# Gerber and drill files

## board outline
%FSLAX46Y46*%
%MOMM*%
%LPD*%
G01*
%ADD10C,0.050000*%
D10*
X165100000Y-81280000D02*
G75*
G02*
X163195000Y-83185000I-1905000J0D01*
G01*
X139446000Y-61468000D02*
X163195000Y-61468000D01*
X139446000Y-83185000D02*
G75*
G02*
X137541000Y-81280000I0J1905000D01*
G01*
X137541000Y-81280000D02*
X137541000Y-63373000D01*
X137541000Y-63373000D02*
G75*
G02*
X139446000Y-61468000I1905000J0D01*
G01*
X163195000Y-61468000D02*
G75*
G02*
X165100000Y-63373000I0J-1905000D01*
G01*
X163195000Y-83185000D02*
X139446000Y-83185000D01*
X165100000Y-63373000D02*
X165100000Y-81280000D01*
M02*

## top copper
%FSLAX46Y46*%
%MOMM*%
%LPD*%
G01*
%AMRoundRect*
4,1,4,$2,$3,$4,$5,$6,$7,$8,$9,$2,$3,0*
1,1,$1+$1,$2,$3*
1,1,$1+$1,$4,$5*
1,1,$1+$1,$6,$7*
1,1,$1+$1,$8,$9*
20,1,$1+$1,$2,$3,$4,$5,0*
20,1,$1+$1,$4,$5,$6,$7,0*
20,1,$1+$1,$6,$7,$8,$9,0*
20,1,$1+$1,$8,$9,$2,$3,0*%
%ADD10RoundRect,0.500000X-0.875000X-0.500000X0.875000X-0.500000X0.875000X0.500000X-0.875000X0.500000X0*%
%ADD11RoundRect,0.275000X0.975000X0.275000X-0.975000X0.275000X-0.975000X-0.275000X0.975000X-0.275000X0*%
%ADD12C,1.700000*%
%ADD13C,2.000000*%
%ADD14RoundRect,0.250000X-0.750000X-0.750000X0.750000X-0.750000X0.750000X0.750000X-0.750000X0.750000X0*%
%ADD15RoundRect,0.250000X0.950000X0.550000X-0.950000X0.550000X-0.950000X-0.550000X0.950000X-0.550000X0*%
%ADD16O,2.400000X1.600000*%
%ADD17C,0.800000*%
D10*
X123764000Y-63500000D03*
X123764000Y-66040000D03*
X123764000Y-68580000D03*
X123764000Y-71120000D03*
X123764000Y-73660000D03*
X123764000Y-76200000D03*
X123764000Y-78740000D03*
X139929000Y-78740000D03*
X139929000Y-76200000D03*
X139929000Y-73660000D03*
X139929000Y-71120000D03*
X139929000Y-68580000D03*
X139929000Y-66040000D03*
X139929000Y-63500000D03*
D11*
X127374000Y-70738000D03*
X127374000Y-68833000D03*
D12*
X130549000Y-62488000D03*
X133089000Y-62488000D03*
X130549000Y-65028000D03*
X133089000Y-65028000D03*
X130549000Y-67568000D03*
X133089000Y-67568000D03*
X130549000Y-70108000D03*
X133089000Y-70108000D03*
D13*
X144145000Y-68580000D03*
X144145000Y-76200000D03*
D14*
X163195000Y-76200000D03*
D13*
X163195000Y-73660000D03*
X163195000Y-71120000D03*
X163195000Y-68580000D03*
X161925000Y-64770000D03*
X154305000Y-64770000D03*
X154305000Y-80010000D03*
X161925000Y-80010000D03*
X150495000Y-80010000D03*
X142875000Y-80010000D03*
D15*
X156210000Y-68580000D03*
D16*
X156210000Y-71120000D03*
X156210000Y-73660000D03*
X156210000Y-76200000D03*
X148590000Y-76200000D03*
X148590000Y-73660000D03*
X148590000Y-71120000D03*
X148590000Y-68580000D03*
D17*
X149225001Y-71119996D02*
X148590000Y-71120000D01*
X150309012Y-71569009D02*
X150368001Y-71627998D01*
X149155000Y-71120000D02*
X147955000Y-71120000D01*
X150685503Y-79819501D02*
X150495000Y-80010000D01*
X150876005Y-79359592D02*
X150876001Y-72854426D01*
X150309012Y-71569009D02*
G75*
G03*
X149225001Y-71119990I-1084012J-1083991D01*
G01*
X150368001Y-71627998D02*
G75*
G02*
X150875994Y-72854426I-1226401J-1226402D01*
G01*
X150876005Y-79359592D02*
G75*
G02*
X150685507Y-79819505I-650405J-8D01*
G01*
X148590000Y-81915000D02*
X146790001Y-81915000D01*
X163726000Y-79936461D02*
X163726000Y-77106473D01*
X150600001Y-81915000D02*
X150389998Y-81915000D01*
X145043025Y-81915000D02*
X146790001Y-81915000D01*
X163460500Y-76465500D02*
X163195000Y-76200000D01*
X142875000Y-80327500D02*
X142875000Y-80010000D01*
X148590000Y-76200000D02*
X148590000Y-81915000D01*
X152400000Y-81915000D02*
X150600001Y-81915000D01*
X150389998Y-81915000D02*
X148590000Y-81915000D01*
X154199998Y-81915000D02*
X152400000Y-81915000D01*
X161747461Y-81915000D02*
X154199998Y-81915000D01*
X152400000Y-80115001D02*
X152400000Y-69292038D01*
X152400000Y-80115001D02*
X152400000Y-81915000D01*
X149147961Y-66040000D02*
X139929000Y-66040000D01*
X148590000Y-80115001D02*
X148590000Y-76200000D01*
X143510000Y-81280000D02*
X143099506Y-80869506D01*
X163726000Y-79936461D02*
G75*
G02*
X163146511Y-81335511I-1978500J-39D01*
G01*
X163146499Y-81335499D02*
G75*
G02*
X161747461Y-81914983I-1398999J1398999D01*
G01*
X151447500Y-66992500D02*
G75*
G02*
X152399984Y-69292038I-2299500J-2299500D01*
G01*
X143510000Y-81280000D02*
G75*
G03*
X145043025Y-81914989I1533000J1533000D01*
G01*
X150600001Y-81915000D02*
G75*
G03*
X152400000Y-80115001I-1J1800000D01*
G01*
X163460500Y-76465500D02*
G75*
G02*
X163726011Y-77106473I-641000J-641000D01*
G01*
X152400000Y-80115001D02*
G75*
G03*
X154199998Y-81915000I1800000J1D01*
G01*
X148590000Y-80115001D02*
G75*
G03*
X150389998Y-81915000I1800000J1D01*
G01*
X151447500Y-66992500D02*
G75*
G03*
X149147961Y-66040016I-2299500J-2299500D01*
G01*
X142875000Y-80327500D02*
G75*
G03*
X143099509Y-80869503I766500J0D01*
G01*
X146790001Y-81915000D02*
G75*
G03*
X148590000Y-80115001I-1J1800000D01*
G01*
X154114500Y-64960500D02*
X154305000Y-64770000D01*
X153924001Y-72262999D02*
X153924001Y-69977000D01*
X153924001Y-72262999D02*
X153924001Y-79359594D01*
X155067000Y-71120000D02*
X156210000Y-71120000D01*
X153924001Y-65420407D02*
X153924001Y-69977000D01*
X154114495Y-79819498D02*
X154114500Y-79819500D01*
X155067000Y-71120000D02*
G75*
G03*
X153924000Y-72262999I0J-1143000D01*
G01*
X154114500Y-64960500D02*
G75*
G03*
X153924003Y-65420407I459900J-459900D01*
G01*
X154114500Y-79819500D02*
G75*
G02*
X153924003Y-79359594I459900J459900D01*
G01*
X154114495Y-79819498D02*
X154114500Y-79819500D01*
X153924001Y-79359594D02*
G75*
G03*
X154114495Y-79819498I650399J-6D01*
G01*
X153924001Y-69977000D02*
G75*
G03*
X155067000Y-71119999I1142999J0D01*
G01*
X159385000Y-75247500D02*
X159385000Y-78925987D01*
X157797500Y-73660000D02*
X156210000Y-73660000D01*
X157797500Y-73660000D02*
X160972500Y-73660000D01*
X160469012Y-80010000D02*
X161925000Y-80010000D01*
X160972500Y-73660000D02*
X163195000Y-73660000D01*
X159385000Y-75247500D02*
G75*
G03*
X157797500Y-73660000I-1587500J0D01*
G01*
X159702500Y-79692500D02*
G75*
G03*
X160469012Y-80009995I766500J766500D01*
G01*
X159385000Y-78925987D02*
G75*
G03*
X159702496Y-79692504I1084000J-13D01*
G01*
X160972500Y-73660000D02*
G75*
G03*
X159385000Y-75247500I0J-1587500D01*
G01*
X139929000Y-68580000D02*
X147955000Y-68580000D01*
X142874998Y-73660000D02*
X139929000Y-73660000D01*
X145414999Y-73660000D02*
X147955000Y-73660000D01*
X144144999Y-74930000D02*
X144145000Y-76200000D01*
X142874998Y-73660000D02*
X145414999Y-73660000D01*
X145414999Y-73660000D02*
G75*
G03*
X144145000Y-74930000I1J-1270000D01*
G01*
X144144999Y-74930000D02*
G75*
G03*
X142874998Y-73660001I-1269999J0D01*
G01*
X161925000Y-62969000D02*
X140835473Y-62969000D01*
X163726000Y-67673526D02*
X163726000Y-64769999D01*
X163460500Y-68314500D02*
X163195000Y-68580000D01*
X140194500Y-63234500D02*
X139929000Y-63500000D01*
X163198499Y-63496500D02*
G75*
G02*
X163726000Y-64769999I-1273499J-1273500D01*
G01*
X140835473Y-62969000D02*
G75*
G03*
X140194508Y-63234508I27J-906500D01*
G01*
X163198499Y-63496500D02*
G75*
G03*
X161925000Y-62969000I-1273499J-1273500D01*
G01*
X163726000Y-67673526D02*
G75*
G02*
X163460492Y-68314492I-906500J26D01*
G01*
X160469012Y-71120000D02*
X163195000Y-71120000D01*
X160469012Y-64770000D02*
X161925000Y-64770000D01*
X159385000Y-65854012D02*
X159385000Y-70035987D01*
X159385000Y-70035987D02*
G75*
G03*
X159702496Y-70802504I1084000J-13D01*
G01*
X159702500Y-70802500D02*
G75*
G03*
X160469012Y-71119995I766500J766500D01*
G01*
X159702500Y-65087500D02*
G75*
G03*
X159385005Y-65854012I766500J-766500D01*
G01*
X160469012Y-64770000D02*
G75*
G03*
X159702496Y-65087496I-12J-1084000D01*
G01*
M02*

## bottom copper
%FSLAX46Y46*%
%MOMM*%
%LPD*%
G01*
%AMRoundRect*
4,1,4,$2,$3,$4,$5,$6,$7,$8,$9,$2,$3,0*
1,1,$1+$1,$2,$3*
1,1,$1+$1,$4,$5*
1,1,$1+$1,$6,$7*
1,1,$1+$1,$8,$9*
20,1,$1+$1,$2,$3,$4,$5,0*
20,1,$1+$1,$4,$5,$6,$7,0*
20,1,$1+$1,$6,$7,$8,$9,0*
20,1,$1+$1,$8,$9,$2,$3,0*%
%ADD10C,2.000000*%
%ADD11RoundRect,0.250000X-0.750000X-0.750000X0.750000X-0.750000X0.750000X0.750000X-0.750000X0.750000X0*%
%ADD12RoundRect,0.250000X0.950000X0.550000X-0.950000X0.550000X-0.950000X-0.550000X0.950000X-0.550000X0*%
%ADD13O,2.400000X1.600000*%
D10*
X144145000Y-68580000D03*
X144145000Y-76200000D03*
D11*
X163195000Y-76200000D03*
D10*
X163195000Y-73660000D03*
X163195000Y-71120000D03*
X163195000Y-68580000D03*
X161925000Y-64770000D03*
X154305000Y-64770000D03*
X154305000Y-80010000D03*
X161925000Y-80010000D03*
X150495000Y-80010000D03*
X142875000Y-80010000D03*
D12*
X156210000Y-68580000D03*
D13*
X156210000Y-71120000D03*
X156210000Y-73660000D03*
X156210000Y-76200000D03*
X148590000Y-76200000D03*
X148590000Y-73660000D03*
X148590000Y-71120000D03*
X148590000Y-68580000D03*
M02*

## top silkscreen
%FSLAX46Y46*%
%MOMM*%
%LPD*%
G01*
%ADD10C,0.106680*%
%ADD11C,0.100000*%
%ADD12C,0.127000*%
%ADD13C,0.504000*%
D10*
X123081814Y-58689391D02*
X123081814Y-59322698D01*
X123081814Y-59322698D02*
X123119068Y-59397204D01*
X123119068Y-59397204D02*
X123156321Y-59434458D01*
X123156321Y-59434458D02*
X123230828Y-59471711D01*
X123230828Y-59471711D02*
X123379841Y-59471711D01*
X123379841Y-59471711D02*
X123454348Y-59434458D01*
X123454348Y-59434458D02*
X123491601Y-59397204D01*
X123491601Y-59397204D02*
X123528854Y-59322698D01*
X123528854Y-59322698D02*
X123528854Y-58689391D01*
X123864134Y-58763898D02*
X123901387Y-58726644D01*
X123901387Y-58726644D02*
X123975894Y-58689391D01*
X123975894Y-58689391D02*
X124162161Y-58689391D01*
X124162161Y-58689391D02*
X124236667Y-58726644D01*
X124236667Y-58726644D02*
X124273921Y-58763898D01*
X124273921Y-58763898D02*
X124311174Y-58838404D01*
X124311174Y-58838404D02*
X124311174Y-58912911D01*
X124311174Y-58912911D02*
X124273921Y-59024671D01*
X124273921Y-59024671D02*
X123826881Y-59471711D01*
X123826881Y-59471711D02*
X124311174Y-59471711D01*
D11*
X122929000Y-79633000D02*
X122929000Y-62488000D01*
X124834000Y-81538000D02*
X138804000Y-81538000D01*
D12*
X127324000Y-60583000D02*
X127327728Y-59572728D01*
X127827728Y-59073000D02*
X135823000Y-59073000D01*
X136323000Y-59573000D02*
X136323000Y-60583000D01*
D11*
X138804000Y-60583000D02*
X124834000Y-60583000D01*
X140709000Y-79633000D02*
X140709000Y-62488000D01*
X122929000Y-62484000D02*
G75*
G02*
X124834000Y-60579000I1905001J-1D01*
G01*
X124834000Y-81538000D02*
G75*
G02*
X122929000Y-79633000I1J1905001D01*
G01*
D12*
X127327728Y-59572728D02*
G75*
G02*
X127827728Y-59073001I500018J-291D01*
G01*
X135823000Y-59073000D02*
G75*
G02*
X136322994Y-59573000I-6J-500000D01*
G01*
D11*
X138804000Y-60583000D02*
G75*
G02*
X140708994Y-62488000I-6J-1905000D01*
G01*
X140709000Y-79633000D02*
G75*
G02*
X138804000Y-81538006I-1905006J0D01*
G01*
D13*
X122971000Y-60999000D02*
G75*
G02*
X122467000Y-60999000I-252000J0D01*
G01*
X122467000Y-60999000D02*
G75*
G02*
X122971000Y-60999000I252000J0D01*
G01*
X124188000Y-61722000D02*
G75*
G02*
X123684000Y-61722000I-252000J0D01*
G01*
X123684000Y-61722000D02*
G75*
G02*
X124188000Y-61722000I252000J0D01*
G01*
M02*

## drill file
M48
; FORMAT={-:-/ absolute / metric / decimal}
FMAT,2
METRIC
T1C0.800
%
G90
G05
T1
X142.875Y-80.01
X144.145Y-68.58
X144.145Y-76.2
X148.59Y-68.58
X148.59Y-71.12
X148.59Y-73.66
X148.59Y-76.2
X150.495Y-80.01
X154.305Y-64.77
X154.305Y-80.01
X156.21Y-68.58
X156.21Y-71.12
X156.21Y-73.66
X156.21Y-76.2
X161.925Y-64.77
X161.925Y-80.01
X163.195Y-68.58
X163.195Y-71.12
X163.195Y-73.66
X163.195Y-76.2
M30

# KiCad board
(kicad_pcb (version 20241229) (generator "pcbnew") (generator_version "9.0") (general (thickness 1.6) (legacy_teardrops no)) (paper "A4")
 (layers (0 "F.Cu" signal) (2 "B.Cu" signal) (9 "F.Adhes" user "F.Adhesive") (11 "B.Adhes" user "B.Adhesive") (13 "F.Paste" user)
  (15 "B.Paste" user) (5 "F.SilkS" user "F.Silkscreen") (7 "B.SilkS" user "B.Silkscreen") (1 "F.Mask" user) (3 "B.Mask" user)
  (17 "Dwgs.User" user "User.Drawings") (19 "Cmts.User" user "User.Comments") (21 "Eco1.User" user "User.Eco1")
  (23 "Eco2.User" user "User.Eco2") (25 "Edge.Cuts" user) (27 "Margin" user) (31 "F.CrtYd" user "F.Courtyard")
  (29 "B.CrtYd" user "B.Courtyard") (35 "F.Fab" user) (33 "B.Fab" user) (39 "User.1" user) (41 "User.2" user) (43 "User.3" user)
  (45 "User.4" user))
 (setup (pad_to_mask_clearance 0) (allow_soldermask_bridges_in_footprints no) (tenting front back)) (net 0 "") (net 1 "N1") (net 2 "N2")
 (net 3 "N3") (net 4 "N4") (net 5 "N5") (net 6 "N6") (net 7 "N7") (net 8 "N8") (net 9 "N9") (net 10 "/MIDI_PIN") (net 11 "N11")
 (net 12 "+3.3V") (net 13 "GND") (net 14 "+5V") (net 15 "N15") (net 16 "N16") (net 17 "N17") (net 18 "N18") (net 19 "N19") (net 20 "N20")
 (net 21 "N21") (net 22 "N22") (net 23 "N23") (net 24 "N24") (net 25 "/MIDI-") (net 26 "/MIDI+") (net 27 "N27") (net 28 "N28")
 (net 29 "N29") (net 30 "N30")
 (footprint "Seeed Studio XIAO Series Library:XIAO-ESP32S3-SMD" (layer "F.Cu") (at 131.825364 71.073)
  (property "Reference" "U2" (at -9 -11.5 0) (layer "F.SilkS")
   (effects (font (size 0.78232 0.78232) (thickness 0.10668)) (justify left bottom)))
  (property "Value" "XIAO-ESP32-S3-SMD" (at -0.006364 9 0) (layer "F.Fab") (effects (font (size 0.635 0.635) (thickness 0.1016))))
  (fp_line (start -8.896364 8.56) (end -8.896364 -8.585) (stroke (width 0.1) (type solid)) (layer "F.SilkS"))
  (fp_line (start -6.991364 10.465) (end 6.978636 10.465) (stroke (width 0.1) (type solid)) (layer "F.SilkS"))
  (fp_line (start -4.501364 -10.49) (end -4.497636 -11.500272) (stroke (width 0.127) (type solid)) (layer "F.SilkS"))
  (fp_line (start -3.997636 -12) (end 3.997636 -12) (stroke (width 0.127) (type solid)) (layer "F.SilkS"))
  (fp_line (start 4.497636 -11.5) (end 4.497636 -10.49) (stroke (width 0.127) (type solid)) (layer "F.SilkS"))
  (fp_line (start 6.978636 -10.49) (end -6.991364 -10.49) (stroke (width 0.1) (type solid)) (layer "F.SilkS"))
  (fp_line (start 8.883636 8.56) (end 8.883636 -8.585) (stroke (width 0.1) (type solid)) (layer "F.SilkS"))
  (fp_arc (start -8.896364 -8.589) (mid -8.338402 -9.936038) (end -6.991364 -10.494) (stroke (width 0.1) (type solid)) (layer "F.SilkS"))
  (fp_arc (start -6.991364 10.465) (mid -8.338402 9.907038) (end -8.896364 8.56) (stroke (width 0.1) (type solid)) (layer "F.SilkS"))
  (fp_arc (start -4.497636 -11.500272) (mid -4.351088 -11.853644) (end -3.997636 -12) (stroke (width 0.127) (type default))
   (layer "F.SilkS"))
  (fp_arc (start 3.997636 -12) (mid 4.351189 -11.853553) (end 4.497636 -11.5) (stroke (width 0.127) (type default)) (layer "F.SilkS"))
  (fp_arc (start 6.978636 -10.49) (mid 8.325674 -9.932038) (end 8.883636 -8.585) (stroke (width 0.1) (type solid)) (layer "F.SilkS"))
  (fp_arc (start 8.883636 8.56) (mid 8.325674 9.907038) (end 6.978636 10.465) (stroke (width 0.1) (type solid)) (layer "F.SilkS"))
  (fp_circle (center -9.106364 -10.074) (end -9.106364 -10.328) (stroke (width 0.5) (type solid)) (fill yes) (layer "F.SilkS"))
  (fp_circle (center -7.889364 -9.351) (end -7.889364 -9.605) (stroke (width 0.5) (type solid)) (fill yes) (layer "F.SilkS"))
  (pad "1" smd roundrect (at -8.061364 -7.573) (size 2.75 2) (layers "F.Cu" "F.Mask" "F.Paste") (roundrect_rratio 0.25) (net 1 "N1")
   (solder_mask_margin 0.0508) (thermal_bridge_angle 45))
  (pad "2" smd roundrect (at -8.061364 -5.033) (size 2.75 2) (layers "F.Cu" "F.Mask" "F.Paste") (roundrect_rratio 0.25) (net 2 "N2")
   (solder_mask_margin 0.0508) (thermal_bridge_angle 45))
  (pad "3" smd roundrect (at -8.061364 -2.493) (size 2.75 2) (layers "F.Cu" "F.Mask" "F.Paste") (roundrect_rratio 0.25) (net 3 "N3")
   (solder_mask_margin 0.0508) (thermal_bridge_angle 45))
  (pad "4" smd roundrect (at -8.061364 0.047) (size 2.75 2) (layers "F.Cu" "F.Mask" "F.Paste") (roundrect_rratio 0.25) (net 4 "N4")
   (solder_mask_margin 0.0508) (thermal_bridge_angle 45))
  (pad "5" smd roundrect (at -8.061364 2.587) (size 2.75 2) (layers "F.Cu" "F.Mask" "F.Paste") (roundrect_rratio 0.25) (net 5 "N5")
   (solder_mask_margin 0.0508) (thermal_bridge_angle 45))
  (pad "6" smd roundrect (at -8.061364 5.127) (size 2.75 2) (layers "F.Cu" "F.Mask" "F.Paste") (roundrect_rratio 0.25) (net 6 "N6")
   (solder_mask_margin 0.0508) (thermal_bridge_angle 45))
  (pad "7" smd roundrect (at -8.061364 7.667) (size 2.75 2) (layers "F.Cu" "F.Mask" "F.Paste") (roundrect_rratio 0.25) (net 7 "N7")
   (solder_mask_margin 0.0508) (thermal_bridge_angle 45))
  (pad "8" smd roundrect (at 8.103636 7.667) (size 2.75 2) (layers "F.Cu" "F.Mask" "F.Paste") (roundrect_rratio 0.25) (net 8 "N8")
   (solder_mask_margin 0.0508) (thermal_bridge_angle 45))
  (pad "9" smd roundrect (at 8.103636 5.127) (size 2.75 2) (layers "F.Cu" "F.Mask" "F.Paste") (roundrect_rratio 0.25) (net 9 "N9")
   (solder_mask_margin 0.0508) (thermal_bridge_angle 45))
  (pad "10" smd roundrect (at 8.103636 2.587) (size 2.75 2) (layers "F.Cu" "F.Mask" "F.Paste") (roundrect_rratio 0.25) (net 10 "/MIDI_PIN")
   (solder_mask_margin 0.0508) (thermal_bridge_angle 45))
  (pad "11" smd roundrect (at 8.103636 0.047) (size 2.75 2) (layers "F.Cu" "F.Mask" "F.Paste") (roundrect_rratio 0.25) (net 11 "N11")
   (solder_mask_margin 0.0508) (thermal_bridge_angle 45))
  (pad "12" smd roundrect (at 8.103636 -2.493) (size 2.75 2) (layers "F.Cu" "F.Mask" "F.Paste") (roundrect_rratio 0.25) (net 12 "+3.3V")
   (solder_mask_margin 0.0508) (thermal_bridge_angle 45))
  (pad "13" smd roundrect (at 8.103636 -5.033) (size 2.75 2) (layers "F.Cu" "F.Mask" "F.Paste") (roundrect_rratio 0.25) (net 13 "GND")
   (solder_mask_margin 0.0508) (thermal_bridge_angle 45))
  (pad "14" smd roundrect (at 8.103636 -7.573) (size 2.75 2) (layers "F.Cu" "F.Mask" "F.Paste") (roundrect_rratio 0.25) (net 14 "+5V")
   (solder_mask_margin 0.0508) (thermal_bridge_angle 45))
  (pad "15" smd roundrect (at -4.451364 -0.335 180) (size 2.5 1.1) (layers "F.Cu" "F.Mask" "F.Paste") (roundrect_rratio 0.25) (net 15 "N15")
   (solder_mask_margin 0.0508) (thermal_bridge_angle 45))
  (pad "16" smd roundrect (at -4.451364 -2.24 180) (size 2.5 1.1) (layers "F.Cu" "F.Mask" "F.Paste") (roundrect_rratio 0.25) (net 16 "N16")
   (solder_mask_margin 0.0508) (thermal_bridge_angle 45))
  (pad "17" smd circle (at -1.276364 -8.585) (size 1.7 1.7) (layers "F.Cu" "F.Mask" "F.Paste") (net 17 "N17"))
  (pad "18" smd circle (at 1.263636 -8.585) (size 1.7 1.7) (layers "F.Cu" "F.Mask" "F.Paste") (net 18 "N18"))
  (pad "19" smd circle (at -1.276364 -6.045) (size 1.7 1.7) (layers "F.Cu" "F.Mask" "F.Paste") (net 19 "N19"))
  (pad "20" smd circle (at 1.263636 -6.045) (size 1.7 1.7) (layers "F.Cu" "F.Mask" "F.Paste") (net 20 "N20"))
  (pad "21" smd circle (at -1.276364 -3.505) (size 1.7 1.7) (layers "F.Cu" "F.Mask" "F.Paste") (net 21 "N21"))
  (pad "22" smd circle (at 1.263636 -3.505) (size 1.7 1.7) (layers "F.Cu" "F.Mask" "F.Paste") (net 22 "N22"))
  (pad "23" smd circle (at -1.276364 -0.965) (size 1.7 1.7) (layers "F.Cu" "F.Mask" "F.Paste") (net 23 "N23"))
  (pad "24" smd circle (at 1.263636 -0.965) (size 1.7 1.7) (layers "F.Cu" "F.Mask" "F.Paste") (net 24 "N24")))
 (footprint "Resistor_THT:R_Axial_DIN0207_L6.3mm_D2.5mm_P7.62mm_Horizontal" (layer "B.Cu") (at 144.145 68.58 -90)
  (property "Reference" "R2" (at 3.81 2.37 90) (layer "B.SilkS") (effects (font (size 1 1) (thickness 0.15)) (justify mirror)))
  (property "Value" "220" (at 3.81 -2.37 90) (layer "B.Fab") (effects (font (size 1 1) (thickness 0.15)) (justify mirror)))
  (pad "1" thru_hole circle (at 0 0 270) (size 2 2) (drill 0.8) (layers "*.Cu" "*.Mask") (remove_unused_layers no) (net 12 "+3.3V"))
  (pad "2" thru_hole circle (at 7.62 0 270) (size 2 2) (drill 0.8) (layers "*.Cu" "*.Mask") (remove_unused_layers no) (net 10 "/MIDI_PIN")))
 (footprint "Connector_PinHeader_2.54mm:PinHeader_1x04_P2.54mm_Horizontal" (layer "B.Cu") (at 163.195 76.2)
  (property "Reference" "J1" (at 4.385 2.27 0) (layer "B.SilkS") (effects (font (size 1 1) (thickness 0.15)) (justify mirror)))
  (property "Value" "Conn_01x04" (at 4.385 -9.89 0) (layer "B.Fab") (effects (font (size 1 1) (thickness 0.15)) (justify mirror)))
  (pad "1" thru_hole roundrect (at 0 0) (size 2 2) (drill 0.8) (layers "*.Cu" "*.Mask") (remove_unused_layers no) (roundrect_rratio 0.125)
   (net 13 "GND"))
  (pad "2" thru_hole circle (at 0 -2.54) (size 2 2) (drill 0.8) (layers "*.Cu" "*.Mask") (remove_unused_layers no) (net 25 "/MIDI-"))
  (pad "3" thru_hole circle (at 0 -5.08) (size 2 2) (drill 0.8) (layers "*.Cu" "*.Mask") (remove_unused_layers no) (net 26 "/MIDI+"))
  (pad "4" thru_hole circle (at 0 -7.62) (size 2 2) (drill 0.8) (layers "*.Cu" "*.Mask") (remove_unused_layers no) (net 14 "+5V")))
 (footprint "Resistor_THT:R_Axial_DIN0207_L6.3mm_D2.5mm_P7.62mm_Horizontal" (layer "B.Cu") (at 161.925 64.77 180)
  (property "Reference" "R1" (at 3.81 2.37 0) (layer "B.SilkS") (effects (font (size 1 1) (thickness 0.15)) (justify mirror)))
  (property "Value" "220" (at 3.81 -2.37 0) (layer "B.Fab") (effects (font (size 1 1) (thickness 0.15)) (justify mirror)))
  (pad "1" thru_hole circle (at 0 0 180) (size 2 2) (drill 0.8) (layers "*.Cu" "*.Mask") (remove_unused_layers no) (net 26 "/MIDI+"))
  (pad "2" thru_hole circle (at 7.62 0 180) (size 2 2) (drill 0.8) (layers "*.Cu" "*.Mask") (remove_unused_layers no) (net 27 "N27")))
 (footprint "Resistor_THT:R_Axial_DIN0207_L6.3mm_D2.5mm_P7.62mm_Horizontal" (layer "B.Cu") (at 154.305 80.01)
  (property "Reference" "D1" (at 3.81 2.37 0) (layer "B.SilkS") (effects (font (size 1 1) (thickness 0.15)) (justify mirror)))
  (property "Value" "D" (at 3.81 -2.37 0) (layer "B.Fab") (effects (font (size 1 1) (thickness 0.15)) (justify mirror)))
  (pad "1" thru_hole circle (at 0 0) (size 2 2) (drill 0.8) (layers "*.Cu" "*.Mask") (remove_unused_layers no) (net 27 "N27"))
  (pad "2" thru_hole circle (at 7.62 0) (size 2 2) (drill 0.8) (layers "*.Cu" "*.Mask") (remove_unused_layers no) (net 25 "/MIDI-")))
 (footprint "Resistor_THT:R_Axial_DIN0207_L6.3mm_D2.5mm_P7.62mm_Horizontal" (layer "B.Cu") (at 150.495 80.01 180)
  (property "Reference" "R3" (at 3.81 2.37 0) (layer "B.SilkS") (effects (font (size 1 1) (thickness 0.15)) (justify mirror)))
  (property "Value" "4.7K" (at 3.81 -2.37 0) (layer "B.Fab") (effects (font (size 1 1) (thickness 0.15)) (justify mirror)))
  (pad "1" thru_hole circle (at 0 0 180) (size 2 2) (drill 0.8) (layers "*.Cu" "*.Mask") (remove_unused_layers no) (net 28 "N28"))
  (pad "2" thru_hole circle (at 7.62 0 180) (size 2 2) (drill 0.8) (layers "*.Cu" "*.Mask") (remove_unused_layers no) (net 13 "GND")))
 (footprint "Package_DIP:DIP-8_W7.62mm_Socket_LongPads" (layer "B.Cu") (at 156.21 68.58 180)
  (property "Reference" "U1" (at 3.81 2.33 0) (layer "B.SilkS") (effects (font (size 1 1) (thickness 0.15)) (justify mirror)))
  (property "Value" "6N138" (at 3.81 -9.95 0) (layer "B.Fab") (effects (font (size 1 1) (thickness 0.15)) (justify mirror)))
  (pad "1" thru_hole roundrect (at 0 0 180) (size 2.4 1.6) (drill 0.8) (layers "*.Cu" "*.Mask") (remove_unused_layers no)
   (roundrect_rratio 0.15625) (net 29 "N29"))
  (pad "2" thru_hole oval (at 0 -2.54 180) (size 2.4 1.6) (drill 0.8) (layers "*.Cu" "*.Mask") (remove_unused_layers no) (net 27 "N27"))
  (pad "3" thru_hole oval (at 0 -5.08 180) (size 2.4 1.6) (drill 0.8) (layers "*.Cu" "*.Mask") (remove_unused_layers no) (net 25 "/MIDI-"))
  (pad "4" thru_hole oval (at 0 -7.62 180) (size 2.4 1.6) (drill 0.8) (layers "*.Cu" "*.Mask") (remove_unused_layers no) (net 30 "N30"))
  (pad "5" thru_hole oval (at 7.62 -7.62 180) (size 2.4 1.6) (drill 0.8) (layers "*.Cu" "*.Mask") (remove_unused_layers no) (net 13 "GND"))
  (pad "6" thru_hole oval (at 7.62 -5.08 180) (size 2.4 1.6) (drill 0.8) (layers "*.Cu" "*.Mask") (remove_unused_layers no)
   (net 10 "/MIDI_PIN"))
  (pad "7" thru_hole oval (at 7.62 -2.54 180) (size 2.4 1.6) (drill 0.8) (layers "*.Cu" "*.Mask") (remove_unused_layers no) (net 28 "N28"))
  (pad "8" thru_hole oval (at 7.62 0 180) (size 2.4 1.6) (drill 0.8) (layers "*.Cu" "*.Mask") (remove_unused_layers no) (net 12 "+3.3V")))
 (gr_arc (start 165.1 81.28) (mid 164.542038 82.627038) (end 163.195 83.185) (stroke (width 0.05) (type default)) (layer "Edge.Cuts"))
 (gr_line (start 139.446 61.468) (end 163.195 61.468) (stroke (width 0.05) (type default)) (layer "Edge.Cuts"))
 (gr_arc (start 139.446 83.185) (mid 138.098962 82.627038) (end 137.541 81.28) (stroke (width 0.05) (type default)) (layer "Edge.Cuts"))
 (gr_line (start 137.541 81.28) (end 137.541 63.373) (stroke (width 0.05) (type default)) (layer "Edge.Cuts"))
 (gr_arc (start 137.541 63.373) (mid 138.098962 62.025962) (end 139.446 61.468) (stroke (width 0.05) (type default)) (layer "Edge.Cuts"))
 (gr_arc (start 163.195 61.468) (mid 164.542038 62.025962) (end 165.1 63.373) (stroke (width 0.05) (type default)) (layer "Edge.Cuts"))
 (gr_line (start 163.195 83.185) (end 139.446 83.185) (stroke (width 0.05) (type default)) (layer "Edge.Cuts"))
 (gr_line (start 165.1 63.373) (end 165.1 81.28) (stroke (width 0.05) (type default)) (layer "Edge.Cuts"))
 (segment (start 149.225001 71.119996) (end 148.59 71.12) (width 0.8) (layer "F.Cu") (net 28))
 (segment (start 150.309012 71.569009) (end 150.368001 71.627998) (width 0.8) (layer "F.Cu") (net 28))
 (segment (start 149.155 71.12) (end 147.955 71.12) (width 0.8) (layer "F.Cu") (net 28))
 (segment (start 150.685503 79.819501) (end 150.495 80.01) (width 0.8) (layer "F.Cu") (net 28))
 (segment (start 150.876005 79.359592) (end 150.876001 72.854426) (width 0.8) (layer "F.Cu") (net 28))
 (arc (start 150.309012 71.569009) (mid 149.811664 71.236689) (end 149.225001 71.119996) (width 0.8) (layer "F.Cu") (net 28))
 (arc (start 150.368001 71.627998) (mid 150.743976 72.190688) (end 150.876001 72.854426) (width 0.8) (layer "F.Cu") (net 28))
 (arc (start 150.876005 79.359592) (mid 150.826495 79.608493) (end 150.685503 79.819501) (width 0.8) (layer "F.Cu") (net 28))
 (segment (start 148.59 81.915) (end 146.790001 81.915) (width 0.8) (layer "F.Cu") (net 13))
 (segment (start 163.726 79.936461) (end 163.726 77.106473) (width 0.8) (layer "F.Cu") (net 13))
 (segment (start 150.600001 81.915) (end 150.389998 81.915) (width 0.8) (layer "F.Cu") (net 13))
 (segment (start 145.043025 81.915) (end 146.790001 81.915) (width 0.8) (layer "F.Cu") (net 13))
 (segment (start 163.4605 76.4655) (end 163.195 76.2) (width 0.8) (layer "F.Cu") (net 13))
 (segment (start 142.875 80.3275) (end 142.875 80.01) (width 0.8) (layer "F.Cu") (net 13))
 (segment (start 148.59 76.2) (end 148.59 81.915) (width 0.8) (layer "F.Cu") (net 13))
 (segment (start 152.4 81.915) (end 150.600001 81.915) (width 0.8) (layer "F.Cu") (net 13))
 (segment (start 150.389998 81.915) (end 148.59 81.915) (width 0.8) (layer "F.Cu") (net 13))
 (segment (start 154.199998 81.915) (end 152.4 81.915) (width 0.8) (layer "F.Cu") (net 13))
 (segment (start 161.747461 81.915) (end 154.199998 81.915) (width 0.8) (layer "F.Cu") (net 13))
 (segment (start 152.4 80.115001) (end 152.4 69.292038) (width 0.8) (layer "F.Cu") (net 13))
 (segment (start 152.4 80.115001) (end 152.4 81.915) (width 0.8) (layer "F.Cu") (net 13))
 (segment (start 149.147961 66.04) (end 139.929 66.04) (width 0.8) (layer "F.Cu") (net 13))
 (segment (start 148.59 80.115001) (end 148.59 76.2) (width 0.8) (layer "F.Cu") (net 13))
 (segment (start 143.51 81.28) (end 143.099506 80.869506) (width 0.8) (layer "F.Cu") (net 13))
 (arc (start 163.726 79.936461) (mid 163.575392 80.693615) (end 163.146499 81.335499) (width 0.8) (layer "F.Cu") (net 13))
 (arc (start 163.146499 81.335499) (mid 162.504615 81.764392) (end 161.747461 81.915) (width 0.8) (layer "F.Cu") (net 13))
 (arc (start 151.4475 66.9925) (mid 152.152453 68.047537) (end 152.4 69.292038) (width 0.8) (layer "F.Cu") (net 13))
 (arc (start 143.51 81.28) (mid 144.213357 81.749968) (end 145.043025 81.915) (width 0.8) (layer "F.Cu") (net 13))
 (arc (start 150.600001 81.915) (mid 151.872792 81.387792) (end 152.4 80.115001) (width 0.8) (layer "F.Cu") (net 13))
 (arc (start 163.4605 76.4655) (mid 163.656998 76.759581) (end 163.726 77.106473) (width 0.8) (layer "F.Cu") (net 13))
 (arc (start 152.4 80.115001) (mid 152.927207 81.387792) (end 154.199998 81.915) (width 0.8) (layer "F.Cu") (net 13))
 (arc (start 148.59 80.115001) (mid 149.117207 81.387792) (end 150.389998 81.915) (width 0.8) (layer "F.Cu") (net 13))
 (arc (start 151.4475 66.9925) (mid 150.392462 66.287546) (end 149.147961 66.04) (width 0.8) (layer "F.Cu") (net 13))
 (arc (start 142.875 80.3275) (mid 142.933347 80.620831) (end 143.099506 80.869506) (width 0.8) (layer "F.Cu") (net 13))
 (arc (start 146.790001 81.915) (mid 148.062792 81.387792) (end 148.59 80.115001) (width 0.8) (layer "F.Cu") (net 13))
 (segment (start 154.1145 64.9605) (end 154.305 64.77) (width 0.8) (layer "F.Cu") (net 27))
 (segment (start 153.924001 72.262999) (end 153.924001 69.977) (width 0.8) (layer "F.Cu") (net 27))
 (segment (start 153.924001 72.262999) (end 153.924001 79.359594) (width 0.8) (layer "F.Cu") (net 27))
 (segment (start 155.067 71.12) (end 156.21 71.12) (width 0.8) (layer "F.Cu") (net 27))
 (segment (start 153.924001 65.420407) (end 153.924001 69.977) (width 0.8) (layer "F.Cu") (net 27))
 (arc (start 154.114495 79.819498) (mid 154.114496 79.819498) (end 154.1145 79.8195) (width 0.8) (layer "F.Cu") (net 27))
 (arc (start 155.067 71.12) (mid 154.258777 71.454776) (end 153.924001 72.262999) (width 0.8) (layer "F.Cu") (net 27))
 (arc (start 154.1145 64.9605) (mid 153.97351 65.171507) (end 153.924001 65.420407) (width 0.8) (layer "F.Cu") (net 27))
 (arc (start 154.1145 79.8195) (mid 153.97351 79.608493) (end 153.924001 79.359594) (width 0.8) (layer "F.Cu") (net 27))
 (arc (start 154.114495 79.819498) (mid 154.114498 79.819499) (end 154.1145 79.8195) (width 0.8) (layer "F.Cu") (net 27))
 (arc (start 153.924001 79.359594) (mid 153.973508 79.608492) (end 154.114495 79.819498) (width 0.8) (layer "F.Cu") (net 27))
 (arc (start 153.924001 69.977) (mid 154.258777 70.785223) (end 155.067 71.12) (width 0.8) (layer "F.Cu") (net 27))
 (segment (start 159.385 75.2475) (end 159.385 78.925987) (width 0.8) (layer "F.Cu") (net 25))
 (segment (start 157.7975 73.66) (end 156.21 73.66) (width 0.8) (layer "F.Cu") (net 25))
 (segment (start 157.7975 73.66) (end 160.9725 73.66) (width 0.8) (layer "F.Cu") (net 25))
 (segment (start 160.469012 80.01) (end 161.925 80.01) (width 0.8) (layer "F.Cu") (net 25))
 (segment (start 160.9725 73.66) (end 163.195 73.66) (width 0.8) (layer "F.Cu") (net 25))
 (arc (start 159.385 75.2475) (mid 158.920032 74.124967) (end 157.7975 73.66) (width 0.8) (layer "F.Cu") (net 25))
 (arc (start 159.7025 79.6925) (mid 160.054178 79.927484) (end 160.469012 80.01) (width 0.8) (layer "F.Cu") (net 25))
 (arc (start 159.385 78.925987) (mid 159.467515 79.34082) (end 159.7025 79.6925) (width 0.8) (layer "F.Cu") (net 25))
 (arc (start 160.9725 73.66) (mid 159.849967 74.124967) (end 159.385 75.2475) (width 0.8) (layer "F.Cu") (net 25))
 (segment (start 139.929 68.58) (end 147.955 68.58) (width 0.8) (layer "F.Cu") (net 12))
 (segment (start 142.874998 73.66) (end 139.929 73.66) (width 0.8) (layer "F.Cu") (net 10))
 (segment (start 145.414999 73.66) (end 147.955 73.66) (width 0.8) (layer "F.Cu") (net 10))
 (segment (start 144.144999 74.93) (end 144.145 76.2) (width 0.8) (layer "F.Cu") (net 10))
 (segment (start 142.874998 73.66) (end 145.414999 73.66) (width 0.8) (layer "F.Cu") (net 10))
 (arc (start 145.414999 73.66) (mid 144.516973 74.031974) (end 144.144999 74.93) (width 0.8) (layer "F.Cu") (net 10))
 (arc (start 144.144999 74.93) (mid 143.773024 74.031974) (end 142.874998 73.66) (width 0.8) (layer "F.Cu") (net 10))
 (segment (start 161.925 62.969) (end 140.835473 62.969) (width 0.8) (layer "F.Cu") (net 14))
 (segment (start 163.726 67.673526) (end 163.726 64.769999) (width 0.8) (layer "F.Cu") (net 14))
 (segment (start 163.4605 68.3145) (end 163.195 68.58) (width 0.8) (layer "F.Cu") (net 14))
 (segment (start 140.1945 63.2345) (end 139.929 63.5) (width 0.8) (layer "F.Cu") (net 14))
 (arc (start 163.198499 63.4965) (mid 163.588906 64.080786) (end 163.726 64.769999) (width 0.8) (layer "F.Cu") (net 14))
 (arc (start 140.835473 62.969) (mid 140.488581 63.038001) (end 140.1945 63.2345) (width 0.8) (layer "F.Cu") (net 14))
 (arc (start 163.198499 63.4965) (mid 162.614212 63.106092) (end 161.925 62.969) (width 0.8) (layer "F.Cu") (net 14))
 (arc (start 163.726 67.673526) (mid 163.656998 68.020418) (end 163.4605 68.3145) (width 0.8) (layer "F.Cu") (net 14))
 (segment (start 160.469012 71.12) (end 163.195 71.12) (width 0.8) (layer "F.Cu") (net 26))
 (segment (start 160.469012 64.77) (end 161.925 64.77) (width 0.8) (layer "F.Cu") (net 26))
 (segment (start 159.385 65.854012) (end 159.385 70.035987) (width 0.8) (layer "F.Cu") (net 26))
 (arc (start 159.385 70.035987) (mid 159.467515 70.45082) (end 159.7025 70.8025) (width 0.8) (layer "F.Cu") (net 26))
 (arc (start 159.7025 70.8025) (mid 160.054178 71.037484) (end 160.469012 71.12) (width 0.8) (layer "F.Cu") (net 26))
 (arc (start 159.7025 65.0875) (mid 159.467515 65.439178) (end 159.385 65.854012) (width 0.8) (layer "F.Cu") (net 26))
 (arc (start 160.469012 64.77) (mid 160.054178 64.852515) (end 159.7025 65.0875) (width 0.8) (layer "F.Cu") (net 26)))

